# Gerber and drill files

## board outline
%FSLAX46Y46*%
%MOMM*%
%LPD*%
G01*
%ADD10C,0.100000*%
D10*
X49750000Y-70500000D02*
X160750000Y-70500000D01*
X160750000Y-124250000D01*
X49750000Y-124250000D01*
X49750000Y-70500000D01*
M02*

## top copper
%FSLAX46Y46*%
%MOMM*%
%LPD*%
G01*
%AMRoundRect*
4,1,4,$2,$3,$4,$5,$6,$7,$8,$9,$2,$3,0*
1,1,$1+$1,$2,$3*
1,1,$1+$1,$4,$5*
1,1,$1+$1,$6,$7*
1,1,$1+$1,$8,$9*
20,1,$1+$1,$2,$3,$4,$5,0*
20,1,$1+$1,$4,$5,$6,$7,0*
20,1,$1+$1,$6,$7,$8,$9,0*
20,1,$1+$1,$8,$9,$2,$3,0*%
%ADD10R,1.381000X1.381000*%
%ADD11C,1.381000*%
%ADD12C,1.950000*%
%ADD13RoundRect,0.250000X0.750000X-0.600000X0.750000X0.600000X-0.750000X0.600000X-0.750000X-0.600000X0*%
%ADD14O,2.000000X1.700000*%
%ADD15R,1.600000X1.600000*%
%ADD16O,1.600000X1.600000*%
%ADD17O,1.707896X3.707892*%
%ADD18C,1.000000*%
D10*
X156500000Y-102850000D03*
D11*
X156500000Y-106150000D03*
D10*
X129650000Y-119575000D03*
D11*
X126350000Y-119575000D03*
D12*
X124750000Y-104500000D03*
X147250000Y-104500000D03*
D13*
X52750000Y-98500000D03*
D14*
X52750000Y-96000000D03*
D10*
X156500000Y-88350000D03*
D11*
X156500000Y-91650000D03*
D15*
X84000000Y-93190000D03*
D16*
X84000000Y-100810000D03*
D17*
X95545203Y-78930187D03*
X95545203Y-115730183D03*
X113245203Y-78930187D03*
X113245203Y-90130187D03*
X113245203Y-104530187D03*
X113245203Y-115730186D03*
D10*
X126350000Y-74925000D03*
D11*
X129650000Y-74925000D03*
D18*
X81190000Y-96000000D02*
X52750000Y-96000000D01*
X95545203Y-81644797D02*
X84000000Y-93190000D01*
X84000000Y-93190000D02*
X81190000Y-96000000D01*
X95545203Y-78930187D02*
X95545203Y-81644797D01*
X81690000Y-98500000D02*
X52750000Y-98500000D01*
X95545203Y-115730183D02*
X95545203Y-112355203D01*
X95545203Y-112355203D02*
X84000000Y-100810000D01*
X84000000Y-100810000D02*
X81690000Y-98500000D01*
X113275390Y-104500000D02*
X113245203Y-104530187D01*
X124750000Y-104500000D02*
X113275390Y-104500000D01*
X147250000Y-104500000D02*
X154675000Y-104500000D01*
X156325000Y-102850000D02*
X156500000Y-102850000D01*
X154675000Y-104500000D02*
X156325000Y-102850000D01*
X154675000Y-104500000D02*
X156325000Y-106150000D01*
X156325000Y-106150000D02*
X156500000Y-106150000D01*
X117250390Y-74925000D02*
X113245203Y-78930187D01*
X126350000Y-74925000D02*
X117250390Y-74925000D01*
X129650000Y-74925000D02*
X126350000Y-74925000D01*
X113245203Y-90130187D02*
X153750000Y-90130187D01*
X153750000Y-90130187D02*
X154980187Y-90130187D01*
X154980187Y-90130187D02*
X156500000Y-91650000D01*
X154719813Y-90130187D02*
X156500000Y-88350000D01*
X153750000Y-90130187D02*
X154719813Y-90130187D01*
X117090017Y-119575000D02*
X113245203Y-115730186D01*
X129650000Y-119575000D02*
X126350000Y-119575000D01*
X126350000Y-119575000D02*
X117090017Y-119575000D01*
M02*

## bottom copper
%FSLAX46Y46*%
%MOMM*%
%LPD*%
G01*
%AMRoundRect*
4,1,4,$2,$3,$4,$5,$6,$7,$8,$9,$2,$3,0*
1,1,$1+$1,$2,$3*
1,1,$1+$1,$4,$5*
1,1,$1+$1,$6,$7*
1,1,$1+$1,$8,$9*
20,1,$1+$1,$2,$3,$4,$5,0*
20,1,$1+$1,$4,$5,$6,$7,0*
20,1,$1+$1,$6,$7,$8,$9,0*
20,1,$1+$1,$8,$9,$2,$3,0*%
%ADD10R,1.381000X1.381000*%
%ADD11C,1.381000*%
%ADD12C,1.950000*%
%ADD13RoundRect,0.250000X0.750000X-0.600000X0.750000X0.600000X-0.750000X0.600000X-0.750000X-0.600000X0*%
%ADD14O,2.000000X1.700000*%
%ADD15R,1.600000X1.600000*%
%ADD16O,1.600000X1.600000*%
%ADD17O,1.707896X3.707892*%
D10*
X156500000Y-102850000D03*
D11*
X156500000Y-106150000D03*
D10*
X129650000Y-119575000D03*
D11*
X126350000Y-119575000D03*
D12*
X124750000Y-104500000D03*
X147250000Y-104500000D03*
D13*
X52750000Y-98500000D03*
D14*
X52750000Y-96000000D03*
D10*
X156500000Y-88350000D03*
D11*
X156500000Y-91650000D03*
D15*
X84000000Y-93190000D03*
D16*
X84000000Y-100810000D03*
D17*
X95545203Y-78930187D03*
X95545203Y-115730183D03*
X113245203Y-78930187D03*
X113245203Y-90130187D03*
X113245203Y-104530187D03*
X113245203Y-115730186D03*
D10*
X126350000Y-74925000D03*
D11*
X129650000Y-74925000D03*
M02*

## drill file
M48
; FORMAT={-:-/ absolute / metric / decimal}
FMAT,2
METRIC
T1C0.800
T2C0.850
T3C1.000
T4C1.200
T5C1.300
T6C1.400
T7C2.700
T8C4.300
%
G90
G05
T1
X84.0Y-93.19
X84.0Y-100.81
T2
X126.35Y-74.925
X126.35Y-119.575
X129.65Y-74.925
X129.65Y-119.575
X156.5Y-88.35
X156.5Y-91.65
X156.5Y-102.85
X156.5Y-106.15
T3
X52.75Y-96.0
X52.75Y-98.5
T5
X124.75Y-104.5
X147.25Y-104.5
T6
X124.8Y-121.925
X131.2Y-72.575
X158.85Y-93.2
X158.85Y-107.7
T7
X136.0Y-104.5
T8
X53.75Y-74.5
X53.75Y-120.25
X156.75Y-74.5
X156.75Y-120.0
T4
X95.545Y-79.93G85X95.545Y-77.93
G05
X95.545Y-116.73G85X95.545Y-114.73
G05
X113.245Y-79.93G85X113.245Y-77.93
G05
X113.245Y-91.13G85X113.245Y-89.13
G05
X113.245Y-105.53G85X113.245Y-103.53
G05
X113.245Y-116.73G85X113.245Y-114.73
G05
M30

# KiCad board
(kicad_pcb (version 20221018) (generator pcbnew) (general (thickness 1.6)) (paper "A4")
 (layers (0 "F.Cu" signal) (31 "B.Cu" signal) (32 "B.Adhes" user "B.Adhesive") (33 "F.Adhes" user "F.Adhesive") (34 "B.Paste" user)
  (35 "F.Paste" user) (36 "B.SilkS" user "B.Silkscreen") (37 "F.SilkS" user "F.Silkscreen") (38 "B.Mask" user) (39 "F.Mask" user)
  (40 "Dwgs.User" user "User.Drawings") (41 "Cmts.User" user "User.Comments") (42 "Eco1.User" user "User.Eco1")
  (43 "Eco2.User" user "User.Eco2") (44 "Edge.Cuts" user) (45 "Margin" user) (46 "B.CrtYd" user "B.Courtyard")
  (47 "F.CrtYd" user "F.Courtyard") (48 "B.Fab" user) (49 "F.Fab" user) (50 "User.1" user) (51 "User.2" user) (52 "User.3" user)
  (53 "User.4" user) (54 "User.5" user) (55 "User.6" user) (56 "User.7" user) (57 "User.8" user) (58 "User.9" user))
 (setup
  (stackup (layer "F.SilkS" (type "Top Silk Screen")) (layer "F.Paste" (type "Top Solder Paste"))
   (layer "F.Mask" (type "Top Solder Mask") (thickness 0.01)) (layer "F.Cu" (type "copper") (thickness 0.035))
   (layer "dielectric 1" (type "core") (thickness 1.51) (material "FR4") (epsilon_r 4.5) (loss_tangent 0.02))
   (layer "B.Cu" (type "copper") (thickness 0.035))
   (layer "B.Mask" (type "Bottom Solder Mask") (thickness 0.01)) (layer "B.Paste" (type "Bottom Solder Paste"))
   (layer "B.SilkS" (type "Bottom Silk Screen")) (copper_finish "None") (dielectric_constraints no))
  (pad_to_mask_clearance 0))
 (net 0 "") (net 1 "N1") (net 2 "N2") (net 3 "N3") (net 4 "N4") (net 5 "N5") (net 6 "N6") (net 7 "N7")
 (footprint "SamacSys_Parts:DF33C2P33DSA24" (layer "F.Cu") (at 156.5 102.85 -90)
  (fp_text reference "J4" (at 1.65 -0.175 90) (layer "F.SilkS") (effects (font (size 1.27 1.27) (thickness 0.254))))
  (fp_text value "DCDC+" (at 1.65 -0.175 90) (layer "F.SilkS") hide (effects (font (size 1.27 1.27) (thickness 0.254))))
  (pad "" np_thru_hole circle (at 4.85 -2.35 270) (size 1.4 1.4) (drill 1.4) (layers "*.Cu" "*.Mask"))
  (pad "1" thru_hole rect (at 0 0 270) (size 1.381 1.381) (drill 0.85) (layers "*.Cu" "*.Mask") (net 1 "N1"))
  (pad "2" thru_hole circle (at 3.3 0 270) (size 1.381 1.381) (drill 0.85) (layers "*.Cu" "*.Mask") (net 1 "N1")))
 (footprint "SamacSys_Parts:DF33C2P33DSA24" (layer "F.Cu") (at 129.65 119.575 180)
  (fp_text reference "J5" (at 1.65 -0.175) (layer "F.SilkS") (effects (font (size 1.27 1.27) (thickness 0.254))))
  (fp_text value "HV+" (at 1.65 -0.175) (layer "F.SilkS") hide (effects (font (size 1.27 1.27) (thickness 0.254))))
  (pad "" np_thru_hole circle (at 4.85 -2.35 180) (size 1.4 1.4) (drill 1.4) (layers "*.Cu" "*.Mask"))
  (pad "1" thru_hole rect (at 0 0 180) (size 1.381 1.381) (drill 0.85) (layers "*.Cu" "*.Mask") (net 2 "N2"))
  (pad "2" thru_hole circle (at 3.3 0 180) (size 1.381 1.381) (drill 0.85) (layers "*.Cu" "*.Mask") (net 2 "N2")))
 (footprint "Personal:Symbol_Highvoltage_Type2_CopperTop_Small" (layer "F.Cu") (at 139.25 90)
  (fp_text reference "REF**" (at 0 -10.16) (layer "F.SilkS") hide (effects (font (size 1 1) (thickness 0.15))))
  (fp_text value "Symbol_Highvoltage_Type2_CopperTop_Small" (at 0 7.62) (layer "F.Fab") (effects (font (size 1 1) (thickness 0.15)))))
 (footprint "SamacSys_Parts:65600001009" (layer "F.Cu") (at 136 104.5)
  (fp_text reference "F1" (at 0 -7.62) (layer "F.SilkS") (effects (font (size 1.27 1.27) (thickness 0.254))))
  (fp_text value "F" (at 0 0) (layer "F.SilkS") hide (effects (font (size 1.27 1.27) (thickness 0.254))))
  (pad "" np_thru_hole circle (at 0 0) (size 2.7 2.7) (drill 2.7) (layers "F&B.Cu" "*.Mask"))
  (pad "1" thru_hole circle (at -11.25 0) (size 1.95 1.95) (drill 1.3) (layers "*.Cu" "*.Mask") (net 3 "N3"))
  (pad "2" thru_hole circle (at 11.25 0) (size 1.95 1.95) (drill 1.3) (layers "*.Cu" "*.Mask") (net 1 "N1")))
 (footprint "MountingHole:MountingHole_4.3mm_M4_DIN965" (layer "F.Cu") (at 156.75 74.5)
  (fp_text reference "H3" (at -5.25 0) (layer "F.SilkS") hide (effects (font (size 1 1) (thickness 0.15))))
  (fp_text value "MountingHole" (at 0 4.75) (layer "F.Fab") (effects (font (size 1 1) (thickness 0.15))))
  (pad "" np_thru_hole circle (at 0 0) (size 4.3 4.3) (drill 4.3) (layers "*.Cu" "*.Mask")))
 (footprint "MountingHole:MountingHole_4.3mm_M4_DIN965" (layer "F.Cu") (at 156.75 120)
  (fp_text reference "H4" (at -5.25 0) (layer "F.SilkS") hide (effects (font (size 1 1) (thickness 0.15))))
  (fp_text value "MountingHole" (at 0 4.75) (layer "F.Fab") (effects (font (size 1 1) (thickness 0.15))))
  (pad "" np_thru_hole circle (at 0 0) (size 4.3 4.3) (drill 4.3) (layers "*.Cu" "*.Mask")))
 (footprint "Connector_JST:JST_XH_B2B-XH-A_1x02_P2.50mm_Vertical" (layer "F.Cu") (at 52.75 98.5 90)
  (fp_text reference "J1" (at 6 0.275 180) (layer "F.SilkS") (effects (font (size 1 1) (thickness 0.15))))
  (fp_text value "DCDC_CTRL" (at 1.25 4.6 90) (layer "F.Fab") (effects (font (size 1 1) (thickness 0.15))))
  (pad "1" thru_hole roundrect (at 0 0 90) (size 1.7 2) (drill 1) (layers "*.Cu" "*.Mask") (roundrect_rratio 0.147059) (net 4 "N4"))
  (pad "2" thru_hole oval (at 2.5 0 90) (size 1.7 2) (drill 1) (layers "*.Cu" "*.Mask") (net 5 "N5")))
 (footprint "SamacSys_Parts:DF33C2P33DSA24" (layer "F.Cu") (at 156.5 88.35 -90)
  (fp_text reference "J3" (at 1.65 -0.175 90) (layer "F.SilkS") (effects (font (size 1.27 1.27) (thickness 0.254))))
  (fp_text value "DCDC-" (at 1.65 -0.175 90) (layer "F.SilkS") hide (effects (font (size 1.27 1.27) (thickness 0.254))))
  (pad "" np_thru_hole circle (at 4.85 -2.35 270) (size 1.4 1.4) (drill 1.4) (layers "*.Cu" "*.Mask"))
  (pad "1" thru_hole rect (at 0 0 270) (size 1.381 1.381) (drill 0.85) (layers "*.Cu" "*.Mask") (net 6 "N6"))
  (pad "2" thru_hole circle (at 3.3 0 270) (size 1.381 1.381) (drill 0.85) (layers "*.Cu" "*.Mask") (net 6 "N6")))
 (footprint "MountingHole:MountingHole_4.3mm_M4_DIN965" (layer "F.Cu") (at 53.75 120.25)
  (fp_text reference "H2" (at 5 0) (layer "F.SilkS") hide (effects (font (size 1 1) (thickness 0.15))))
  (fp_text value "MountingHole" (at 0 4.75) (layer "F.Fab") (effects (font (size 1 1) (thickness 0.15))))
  (pad "" np_thru_hole circle (at 0 0) (size 4.3 4.3) (drill 4.3) (layers "*.Cu" "*.Mask")))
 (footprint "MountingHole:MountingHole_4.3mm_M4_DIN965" (layer "F.Cu") (at 53.75 74.5)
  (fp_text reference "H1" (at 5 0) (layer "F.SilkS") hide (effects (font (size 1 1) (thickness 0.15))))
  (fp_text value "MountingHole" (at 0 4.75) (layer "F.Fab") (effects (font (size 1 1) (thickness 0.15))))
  (pad "" np_thru_hole circle (at 0 0) (size 4.3 4.3) (drill 4.3) (layers "*.Cu" "*.Mask")))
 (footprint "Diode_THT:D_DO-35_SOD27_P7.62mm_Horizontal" (layer "F.Cu") (at 84 93.19 -90)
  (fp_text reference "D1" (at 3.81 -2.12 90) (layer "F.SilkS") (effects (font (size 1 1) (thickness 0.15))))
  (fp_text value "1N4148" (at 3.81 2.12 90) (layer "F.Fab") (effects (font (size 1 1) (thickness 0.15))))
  (pad "1" thru_hole rect (at 0 0 270) (size 1.6 1.6) (drill 0.8) (layers "*.Cu" "*.Mask") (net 5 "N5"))
  (pad "2" thru_hole oval (at 7.62 0 270) (size 1.6 1.6) (drill 0.8) (layers "*.Cu" "*.Mask") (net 4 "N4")))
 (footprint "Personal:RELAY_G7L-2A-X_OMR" (layer "F.Cu") (at 95.545203 78.930187)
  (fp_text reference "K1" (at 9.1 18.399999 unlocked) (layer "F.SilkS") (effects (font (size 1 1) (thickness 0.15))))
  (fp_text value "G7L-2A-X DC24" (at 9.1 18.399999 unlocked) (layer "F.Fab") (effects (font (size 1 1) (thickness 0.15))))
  (pad "0" thru_hole oval (at 0 0 90) (size 3.707892 1.707896) (drill oval 3.2 1.2) (layers "*.Cu" "*.Mask") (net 5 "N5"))
  (pad "1" thru_hole oval (at 0 36.799996 90) (size 3.707892 1.707896) (drill oval 3.2 1.2) (layers "*.Cu" "*.Mask") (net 4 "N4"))
  (pad "2" thru_hole oval (at 17.7 0 90) (size 3.707892 1.707896) (drill oval 3.2 1.2) (layers "*.Cu" "*.Mask") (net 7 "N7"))
  (pad "4" thru_hole oval (at 17.7 11.2 90) (size 3.707892 1.707896) (drill oval 3.2 1.2) (layers "*.Cu" "*.Mask") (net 6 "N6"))
  (pad "6" thru_hole oval (at 17.7 25.6 90) (size 3.707892 1.707896) (drill oval 3.2 1.2) (layers "*.Cu" "*.Mask") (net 3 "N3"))
  (pad "8" thru_hole oval (at 17.7 36.799999 90) (size 3.707892 1.707896) (drill oval 3.2 1.2) (layers "*.Cu" "*.Mask") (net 2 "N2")))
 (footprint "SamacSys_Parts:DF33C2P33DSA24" (layer "F.Cu") (at 126.35 74.925)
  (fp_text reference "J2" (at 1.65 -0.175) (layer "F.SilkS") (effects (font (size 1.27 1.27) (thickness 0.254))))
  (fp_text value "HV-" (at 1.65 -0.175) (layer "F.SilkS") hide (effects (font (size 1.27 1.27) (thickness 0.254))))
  (pad "" np_thru_hole circle (at 4.85 -2.35) (size 1.4 1.4) (drill 1.4) (layers "*.Cu" "*.Mask"))
  (pad "1" thru_hole rect (at 0 0) (size 1.381 1.381) (drill 0.85) (layers "*.Cu" "*.Mask") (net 7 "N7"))
  (pad "2" thru_hole circle (at 3.3 0) (size 1.381 1.381) (drill 0.85) (layers "*.Cu" "*.Mask") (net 7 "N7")))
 (gr_rect (start 49.75 70.5) (end 160.75 124.25) (stroke (width 0.1) (type default)) (fill none) (layer "Edge.Cuts"))
 (segment (start 81.19 96) (end 52.75 96) (width 1) (layer "F.Cu") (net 5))
 (segment (start 95.545203 81.644797) (end 84 93.19) (width 1) (layer "F.Cu") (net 5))
 (segment (start 84 93.19) (end 81.19 96) (width 1) (layer "F.Cu") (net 5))
 (segment (start 95.545203 78.930187) (end 95.545203 81.644797) (width 1) (layer "F.Cu") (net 5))
 (segment (start 81.69 98.5) (end 52.75 98.5) (width 1) (layer "F.Cu") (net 4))
 (segment (start 95.545203 115.730183) (end 95.545203 112.355203) (width 1) (layer "F.Cu") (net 4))
 (segment (start 95.545203 112.355203) (end 84 100.81) (width 1) (layer "F.Cu") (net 4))
 (segment (start 84 100.81) (end 81.69 98.5) (width 1) (layer "F.Cu") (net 4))
 (segment (start 113.27539 104.5) (end 113.245203 104.530187) (width 1) (layer "F.Cu") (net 3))
 (segment (start 124.75 104.5) (end 113.27539 104.5) (width 1) (layer "F.Cu") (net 3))
 (segment (start 147.25 104.5) (end 154.675 104.5) (width 1) (layer "F.Cu") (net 1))
 (segment (start 156.325 102.85) (end 156.5 102.85) (width 1) (layer "F.Cu") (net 1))
 (segment (start 154.675 104.5) (end 156.325 102.85) (width 1) (layer "F.Cu") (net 1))
 (segment (start 154.675 104.5) (end 156.325 106.15) (width 1) (layer "F.Cu") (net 1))
 (segment (start 156.325 106.15) (end 156.5 106.15) (width 1) (layer "F.Cu") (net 1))
 (segment (start 117.25039 74.925) (end 113.245203 78.930187) (width 1) (layer "F.Cu") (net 7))
 (segment (start 126.35 74.925) (end 117.25039 74.925) (width 1) (layer "F.Cu") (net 7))
 (segment (start 129.65 74.925) (end 126.35 74.925) (width 1) (layer "F.Cu") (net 7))
 (segment (start 113.245203 90.130187) (end 153.75 90.130187) (width 1) (layer "F.Cu") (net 6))
 (segment (start 153.75 90.130187) (end 154.980187 90.130187) (width 1) (layer "F.Cu") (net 6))
 (segment (start 154.980187 90.130187) (end 156.5 91.65) (width 1) (layer "F.Cu") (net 6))
 (segment (start 154.719813 90.130187) (end 156.5 88.35) (width 1) (layer "F.Cu") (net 6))
 (segment (start 153.75 90.130187) (end 154.719813 90.130187) (width 1) (layer "F.Cu") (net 6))
 (segment (start 117.090017 119.575) (end 113.245203 115.730186) (width 1) (layer "F.Cu") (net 2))
 (segment (start 129.65 119.575) (end 126.35 119.575) (width 1) (layer "F.Cu") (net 2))
 (segment (start 126.35 119.575) (end 117.090017 119.575) (width 1) (layer "F.Cu") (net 2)))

